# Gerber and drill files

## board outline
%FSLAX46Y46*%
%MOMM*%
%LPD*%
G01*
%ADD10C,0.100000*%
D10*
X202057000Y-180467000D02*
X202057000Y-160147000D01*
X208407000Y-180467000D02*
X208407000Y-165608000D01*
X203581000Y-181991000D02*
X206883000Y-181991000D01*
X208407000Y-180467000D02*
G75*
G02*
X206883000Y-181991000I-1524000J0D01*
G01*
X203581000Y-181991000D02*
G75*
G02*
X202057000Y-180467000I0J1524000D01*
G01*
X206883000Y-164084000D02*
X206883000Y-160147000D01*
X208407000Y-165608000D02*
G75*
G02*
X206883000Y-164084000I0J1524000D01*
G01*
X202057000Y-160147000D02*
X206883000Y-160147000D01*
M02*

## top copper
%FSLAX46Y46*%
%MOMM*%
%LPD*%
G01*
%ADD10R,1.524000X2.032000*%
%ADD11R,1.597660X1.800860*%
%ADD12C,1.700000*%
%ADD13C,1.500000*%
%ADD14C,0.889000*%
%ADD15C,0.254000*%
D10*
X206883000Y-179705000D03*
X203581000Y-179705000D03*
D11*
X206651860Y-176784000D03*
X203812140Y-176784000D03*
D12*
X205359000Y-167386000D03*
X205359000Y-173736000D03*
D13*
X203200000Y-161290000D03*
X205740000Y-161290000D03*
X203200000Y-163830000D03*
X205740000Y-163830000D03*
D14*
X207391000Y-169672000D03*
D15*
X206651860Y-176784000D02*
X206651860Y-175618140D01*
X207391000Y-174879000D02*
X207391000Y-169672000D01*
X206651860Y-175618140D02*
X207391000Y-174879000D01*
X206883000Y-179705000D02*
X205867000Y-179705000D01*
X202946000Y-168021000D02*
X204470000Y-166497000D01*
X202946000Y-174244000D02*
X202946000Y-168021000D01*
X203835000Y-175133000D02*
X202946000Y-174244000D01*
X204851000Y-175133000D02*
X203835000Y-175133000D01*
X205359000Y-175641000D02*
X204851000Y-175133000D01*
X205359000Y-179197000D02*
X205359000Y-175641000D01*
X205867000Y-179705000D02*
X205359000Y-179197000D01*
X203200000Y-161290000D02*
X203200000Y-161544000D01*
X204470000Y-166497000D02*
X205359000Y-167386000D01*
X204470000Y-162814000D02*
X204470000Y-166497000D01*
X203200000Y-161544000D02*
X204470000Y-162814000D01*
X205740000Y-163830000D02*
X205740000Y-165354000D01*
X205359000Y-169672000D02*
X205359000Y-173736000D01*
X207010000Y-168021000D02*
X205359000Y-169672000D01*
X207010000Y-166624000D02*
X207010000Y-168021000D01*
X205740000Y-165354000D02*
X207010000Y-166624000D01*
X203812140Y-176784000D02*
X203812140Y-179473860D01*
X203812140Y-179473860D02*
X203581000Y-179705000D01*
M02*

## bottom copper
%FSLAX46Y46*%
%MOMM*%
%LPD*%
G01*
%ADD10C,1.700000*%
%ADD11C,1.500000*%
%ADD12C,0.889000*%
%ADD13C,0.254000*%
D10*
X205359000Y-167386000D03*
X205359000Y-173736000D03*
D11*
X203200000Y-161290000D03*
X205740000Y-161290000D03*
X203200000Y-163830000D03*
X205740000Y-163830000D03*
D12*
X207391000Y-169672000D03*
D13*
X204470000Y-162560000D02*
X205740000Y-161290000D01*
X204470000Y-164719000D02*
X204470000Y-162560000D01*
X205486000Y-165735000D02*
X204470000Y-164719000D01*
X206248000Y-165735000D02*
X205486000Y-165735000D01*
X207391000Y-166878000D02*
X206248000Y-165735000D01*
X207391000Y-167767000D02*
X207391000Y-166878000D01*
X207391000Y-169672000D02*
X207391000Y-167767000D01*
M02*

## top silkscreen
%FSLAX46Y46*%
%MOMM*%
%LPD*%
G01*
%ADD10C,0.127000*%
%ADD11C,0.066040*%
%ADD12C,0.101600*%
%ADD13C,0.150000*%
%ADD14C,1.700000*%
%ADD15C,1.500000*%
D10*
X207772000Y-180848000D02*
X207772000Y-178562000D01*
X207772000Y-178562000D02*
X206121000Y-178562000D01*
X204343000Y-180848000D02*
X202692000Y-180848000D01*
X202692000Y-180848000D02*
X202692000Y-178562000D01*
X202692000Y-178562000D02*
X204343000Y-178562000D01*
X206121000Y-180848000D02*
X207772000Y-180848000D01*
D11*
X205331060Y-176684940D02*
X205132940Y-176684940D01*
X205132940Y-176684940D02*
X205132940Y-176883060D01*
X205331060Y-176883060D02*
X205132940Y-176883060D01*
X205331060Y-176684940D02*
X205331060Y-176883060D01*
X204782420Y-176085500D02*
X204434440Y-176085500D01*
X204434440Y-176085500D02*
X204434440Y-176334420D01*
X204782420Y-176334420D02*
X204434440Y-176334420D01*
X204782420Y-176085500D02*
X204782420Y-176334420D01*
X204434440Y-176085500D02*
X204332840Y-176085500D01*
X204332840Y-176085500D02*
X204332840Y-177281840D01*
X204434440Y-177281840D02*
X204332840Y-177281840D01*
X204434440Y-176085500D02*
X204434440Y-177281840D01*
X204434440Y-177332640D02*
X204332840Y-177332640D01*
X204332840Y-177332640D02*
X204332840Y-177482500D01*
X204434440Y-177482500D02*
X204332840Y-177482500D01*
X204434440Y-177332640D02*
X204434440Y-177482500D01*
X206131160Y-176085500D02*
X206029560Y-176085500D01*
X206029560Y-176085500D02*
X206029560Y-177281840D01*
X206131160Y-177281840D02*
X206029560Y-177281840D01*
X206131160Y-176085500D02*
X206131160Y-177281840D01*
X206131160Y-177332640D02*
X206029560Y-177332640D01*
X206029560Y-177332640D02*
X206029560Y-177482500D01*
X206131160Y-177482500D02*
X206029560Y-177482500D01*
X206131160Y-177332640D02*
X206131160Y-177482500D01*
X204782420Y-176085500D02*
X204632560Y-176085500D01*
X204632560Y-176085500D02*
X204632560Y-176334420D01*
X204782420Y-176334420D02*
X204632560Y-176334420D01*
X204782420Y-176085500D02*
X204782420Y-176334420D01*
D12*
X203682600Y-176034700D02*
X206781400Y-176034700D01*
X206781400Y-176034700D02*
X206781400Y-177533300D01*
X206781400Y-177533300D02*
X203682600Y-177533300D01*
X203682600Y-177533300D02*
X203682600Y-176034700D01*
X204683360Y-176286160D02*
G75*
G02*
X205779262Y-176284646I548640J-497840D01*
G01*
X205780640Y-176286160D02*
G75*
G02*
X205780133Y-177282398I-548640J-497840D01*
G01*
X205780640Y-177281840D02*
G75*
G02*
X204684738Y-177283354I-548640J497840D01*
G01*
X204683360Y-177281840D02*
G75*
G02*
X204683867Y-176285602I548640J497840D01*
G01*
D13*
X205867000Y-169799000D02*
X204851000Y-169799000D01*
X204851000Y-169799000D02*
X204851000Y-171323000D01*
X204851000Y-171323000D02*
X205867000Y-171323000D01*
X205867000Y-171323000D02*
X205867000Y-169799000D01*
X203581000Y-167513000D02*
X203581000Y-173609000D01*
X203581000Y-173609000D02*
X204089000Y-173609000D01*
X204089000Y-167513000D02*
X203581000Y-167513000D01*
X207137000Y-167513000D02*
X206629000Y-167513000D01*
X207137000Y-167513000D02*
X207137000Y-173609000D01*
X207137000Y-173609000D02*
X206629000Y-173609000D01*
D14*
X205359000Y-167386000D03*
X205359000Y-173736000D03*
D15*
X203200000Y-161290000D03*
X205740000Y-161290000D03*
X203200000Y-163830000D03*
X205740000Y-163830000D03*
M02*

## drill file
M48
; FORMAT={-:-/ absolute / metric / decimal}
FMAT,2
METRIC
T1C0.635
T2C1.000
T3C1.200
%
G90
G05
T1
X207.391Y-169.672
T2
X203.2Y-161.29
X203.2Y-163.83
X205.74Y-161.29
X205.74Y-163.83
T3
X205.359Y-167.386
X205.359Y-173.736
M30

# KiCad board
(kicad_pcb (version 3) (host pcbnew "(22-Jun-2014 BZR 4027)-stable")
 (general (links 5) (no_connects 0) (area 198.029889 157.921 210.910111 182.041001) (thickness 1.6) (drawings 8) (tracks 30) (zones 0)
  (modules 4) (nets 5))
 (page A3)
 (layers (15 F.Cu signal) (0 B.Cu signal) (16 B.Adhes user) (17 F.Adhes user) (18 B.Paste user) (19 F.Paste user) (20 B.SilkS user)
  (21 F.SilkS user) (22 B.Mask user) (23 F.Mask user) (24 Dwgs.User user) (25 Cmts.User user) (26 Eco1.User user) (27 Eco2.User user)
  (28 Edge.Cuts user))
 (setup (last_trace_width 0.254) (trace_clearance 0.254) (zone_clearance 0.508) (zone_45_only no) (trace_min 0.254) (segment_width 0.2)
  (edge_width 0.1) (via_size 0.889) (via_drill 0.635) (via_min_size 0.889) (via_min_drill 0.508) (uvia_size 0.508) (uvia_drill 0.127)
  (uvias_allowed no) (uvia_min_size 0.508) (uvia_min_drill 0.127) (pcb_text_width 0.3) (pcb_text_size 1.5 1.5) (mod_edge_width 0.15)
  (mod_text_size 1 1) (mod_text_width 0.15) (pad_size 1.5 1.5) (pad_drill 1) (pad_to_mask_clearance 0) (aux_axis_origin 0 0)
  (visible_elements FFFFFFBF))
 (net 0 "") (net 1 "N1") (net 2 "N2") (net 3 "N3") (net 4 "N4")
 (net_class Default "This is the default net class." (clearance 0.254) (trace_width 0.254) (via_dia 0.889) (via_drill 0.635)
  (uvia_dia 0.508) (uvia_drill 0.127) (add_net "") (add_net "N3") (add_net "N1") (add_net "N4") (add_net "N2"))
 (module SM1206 (layer F.Cu) (at 205.232 179.705 180)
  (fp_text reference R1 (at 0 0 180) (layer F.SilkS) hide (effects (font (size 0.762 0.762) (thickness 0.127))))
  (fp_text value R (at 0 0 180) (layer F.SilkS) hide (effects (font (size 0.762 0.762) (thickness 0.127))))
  (fp_line (start -2.54 -1.143) (end -2.54 1.143) (layer F.SilkS) (width 0.127))
  (fp_line (start -2.54 1.143) (end -0.889 1.143) (layer F.SilkS) (width 0.127))
  (fp_line (start 0.889 -1.143) (end 2.54 -1.143) (layer F.SilkS) (width 0.127))
  (fp_line (start 2.54 -1.143) (end 2.54 1.143) (layer F.SilkS) (width 0.127))
  (fp_line (start 2.54 1.143) (end 0.889 1.143) (layer F.SilkS) (width 0.127))
  (fp_line (start -0.889 -1.143) (end -2.54 -1.143) (layer F.SilkS) (width 0.127))
  (pad 1 smd rect (at -1.651 0 180) (size 1.524 2.032) (layers F.Cu F.Paste F.Mask) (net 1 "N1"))
  (pad 2 smd rect (at 1.651 0 180) (size 1.524 2.032) (layers F.Cu F.Paste F.Mask) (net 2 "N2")))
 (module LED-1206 (layer F.Cu) (at 205.232 176.784 180)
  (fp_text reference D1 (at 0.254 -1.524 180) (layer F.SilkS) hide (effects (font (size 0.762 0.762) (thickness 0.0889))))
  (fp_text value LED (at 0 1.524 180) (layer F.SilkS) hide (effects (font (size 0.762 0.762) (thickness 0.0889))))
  (fp_line (start -0.09906 0.09906) (end 0.09906 0.09906) (layer F.SilkS) (width 0.06604))
  (fp_line (start 0.09906 0.09906) (end 0.09906 -0.09906) (layer F.SilkS) (width 0.06604))
  (fp_line (start -0.09906 -0.09906) (end 0.09906 -0.09906) (layer F.SilkS) (width 0.06604))
  (fp_line (start -0.09906 0.09906) (end -0.09906 -0.09906) (layer F.SilkS) (width 0.06604))
  (fp_line (start 0.44958 0.6985) (end 0.79756 0.6985) (layer F.SilkS) (width 0.06604))
  (fp_line (start 0.79756 0.6985) (end 0.79756 0.44958) (layer F.SilkS) (width 0.06604))
  (fp_line (start 0.44958 0.44958) (end 0.79756 0.44958) (layer F.SilkS) (width 0.06604))
  (fp_line (start 0.44958 0.6985) (end 0.44958 0.44958) (layer F.SilkS) (width 0.06604))
  (fp_line (start 0.79756 0.6985) (end 0.89916 0.6985) (layer F.SilkS) (width 0.06604))
  (fp_line (start 0.89916 0.6985) (end 0.89916 -0.49784) (layer F.SilkS) (width 0.06604))
  (fp_line (start 0.79756 -0.49784) (end 0.89916 -0.49784) (layer F.SilkS) (width 0.06604))
  (fp_line (start 0.79756 0.6985) (end 0.79756 -0.49784) (layer F.SilkS) (width 0.06604))
  (fp_line (start 0.79756 -0.54864) (end 0.89916 -0.54864) (layer F.SilkS) (width 0.06604))
  (fp_line (start 0.89916 -0.54864) (end 0.89916 -0.6985) (layer F.SilkS) (width 0.06604))
  (fp_line (start 0.79756 -0.6985) (end 0.89916 -0.6985) (layer F.SilkS) (width 0.06604))
  (fp_line (start 0.79756 -0.54864) (end 0.79756 -0.6985) (layer F.SilkS) (width 0.06604))
  (fp_line (start -0.89916 0.6985) (end -0.79756 0.6985) (layer F.SilkS) (width 0.06604))
  (fp_line (start -0.79756 0.6985) (end -0.79756 -0.49784) (layer F.SilkS) (width 0.06604))
  (fp_line (start -0.89916 -0.49784) (end -0.79756 -0.49784) (layer F.SilkS) (width 0.06604))
  (fp_line (start -0.89916 0.6985) (end -0.89916 -0.49784) (layer F.SilkS) (width 0.06604))
  (fp_line (start -0.89916 -0.54864) (end -0.79756 -0.54864) (layer F.SilkS) (width 0.06604))
  (fp_line (start -0.79756 -0.54864) (end -0.79756 -0.6985) (layer F.SilkS) (width 0.06604))
  (fp_line (start -0.89916 -0.6985) (end -0.79756 -0.6985) (layer F.SilkS) (width 0.06604))
  (fp_line (start -0.89916 -0.54864) (end -0.89916 -0.6985) (layer F.SilkS) (width 0.06604))
  (fp_line (start 0.44958 0.6985) (end 0.59944 0.6985) (layer F.SilkS) (width 0.06604))
  (fp_line (start 0.59944 0.6985) (end 0.59944 0.44958) (layer F.SilkS) (width 0.06604))
  (fp_line (start 0.44958 0.44958) (end 0.59944 0.44958) (layer F.SilkS) (width 0.06604))
  (fp_line (start 0.44958 0.6985) (end 0.44958 0.44958) (layer F.SilkS) (width 0.06604))
  (fp_line (start 1.5494 0.7493) (end -1.5494 0.7493) (layer F.SilkS) (width 0.1016))
  (fp_line (start -1.5494 0.7493) (end -1.5494 -0.7493) (layer F.SilkS) (width 0.1016))
  (fp_line (start -1.5494 -0.7493) (end 1.5494 -0.7493) (layer F.SilkS) (width 0.1016))
  (fp_line (start 1.5494 -0.7493) (end 1.5494 0.7493) (layer F.SilkS) (width 0.1016))
  (fp_arc (start 0 0) (end 0.54864 0.49784) (angle 95.4) (layer F.SilkS) (width 0.1016))
  (fp_arc (start 0 0) (end -0.54864 0.49784) (angle 84.5) (layer F.SilkS) (width 0.1016))
  (fp_arc (start 0 0) (end -0.54864 -0.49784) (angle 95.4) (layer F.SilkS) (width 0.1016))
  (fp_arc (start 0 0) (end 0.54864 -0.49784) (angle 84.5) (layer F.SilkS) (width 0.1016))
  (pad 1 smd rect (at -1.41986 0 180) (size 1.59766 1.80086) (layers F.Cu F.Paste F.Mask) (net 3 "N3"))
  (pad 2 smd rect (at 1.41986 0 180) (size 1.59766 1.80086) (layers F.Cu F.Paste F.Mask) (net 2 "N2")))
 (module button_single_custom (layer F.Cu) (at 205.359 170.561 270)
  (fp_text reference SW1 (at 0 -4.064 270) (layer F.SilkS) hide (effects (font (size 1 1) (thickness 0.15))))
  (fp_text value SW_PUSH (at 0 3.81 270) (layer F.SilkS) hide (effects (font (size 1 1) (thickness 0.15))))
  (fp_line (start -0.762 -0.508) (end -0.762 0.508) (layer F.SilkS) (width 0.15))
  (fp_line (start -0.762 0.508) (end 0.762 0.508) (layer F.SilkS) (width 0.15))
  (fp_line (start 0.762 0.508) (end 0.762 -0.508) (layer F.SilkS) (width 0.15))
  (fp_line (start 0.762 -0.508) (end -0.762 -0.508) (layer F.SilkS) (width 0.15))
  (fp_line (start -3.048 1.778) (end 3.048 1.778) (layer F.SilkS) (width 0.15))
  (fp_line (start 3.048 1.778) (end 3.048 1.27) (layer F.SilkS) (width 0.15))
  (fp_line (start -3.048 1.27) (end -3.048 1.778) (layer F.SilkS) (width 0.15))
  (fp_line (start -3.048 -1.778) (end -3.048 -1.27) (layer F.SilkS) (width 0.15))
  (fp_line (start -3.048 -1.778) (end 3.048 -1.778) (layer F.SilkS) (width 0.15))
  (fp_line (start 3.048 -1.778) (end 3.048 -1.27) (layer F.SilkS) (width 0.15))
  (pad 1 thru_hole circle (at -3.175 0 270) (size 1.7 1.7) (drill 1.2) (layers *.Cu *.Mask F.SilkS) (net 1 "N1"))
  (pad 2 thru_hole circle (at 3.175 0 270) (size 1.7 1.7) (drill 1.2) (layers *.Cu *.Mask F.SilkS) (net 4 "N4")))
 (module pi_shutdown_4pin (layer F.Cu) (at 204.47 162.56)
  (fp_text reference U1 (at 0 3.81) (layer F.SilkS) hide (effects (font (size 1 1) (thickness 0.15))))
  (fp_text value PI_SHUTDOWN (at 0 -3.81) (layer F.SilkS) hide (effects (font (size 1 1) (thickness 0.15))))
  (pad 14 thru_hole circle (at -1.27 -1.27) (size 1.5 1.5) (drill 1) (layers *.Cu *.Mask F.SilkS) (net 1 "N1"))
  (pad 16 thru_hole circle (at 1.27 -1.27) (size 1.5 1.5) (drill 1) (layers *.Cu *.Mask F.SilkS) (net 3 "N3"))
  (pad 13 thru_hole circle (at -1.27 1.27) (size 1.5 1.5) (drill 1) (layers *.Cu *.Mask F.SilkS))
  (pad 15 thru_hole circle (at 1.27 1.27) (size 1.5 1.5) (drill 1) (layers *.Cu *.Mask F.SilkS) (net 4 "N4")))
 (gr_line (start 202.057 180.467) (end 202.057 160.147) (angle 90) (layer Edge.Cuts) (width 0.1))
 (gr_line (start 208.407 180.467) (end 208.407 165.608) (angle 90) (layer Edge.Cuts) (width 0.1))
 (gr_line (start 203.581 181.991) (end 206.883 181.991) (angle 90) (layer Edge.Cuts) (width 0.1))
 (gr_arc (start 206.883 180.467) (end 208.407 180.467) (angle 90) (layer Edge.Cuts) (width 0.1))
 (gr_arc (start 203.581 180.467) (end 203.581 181.991) (angle 90) (layer Edge.Cuts) (width 0.1))
 (gr_line (start 206.883 164.084) (end 206.883 160.147) (angle 90) (layer Edge.Cuts) (width 0.1))
 (gr_arc (start 208.407 164.084) (end 208.407 165.608) (angle 90) (layer Edge.Cuts) (width 0.1))
 (gr_line (start 202.057 160.147) (end 206.883 160.147) (angle 90) (layer Edge.Cuts) (width 0.1))
 (segment (start 206.65186 176.784) (end 206.65186 175.61814) (width 0.254) (layer F.Cu) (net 3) (status 400000))
 (segment (start 204.47 162.56) (end 205.74 161.29) (width 0.254) (layer B.Cu) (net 3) (status 800000))
 (segment (start 204.47 164.719) (end 204.47 162.56) (width 0.254) (layer B.Cu) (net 3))
 (segment (start 205.486 165.735) (end 204.47 164.719) (width 0.254) (layer B.Cu) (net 3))
 (segment (start 206.248 165.735) (end 205.486 165.735) (width 0.254) (layer B.Cu) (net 3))
 (segment (start 207.391 166.878) (end 206.248 165.735) (width 0.254) (layer B.Cu) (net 3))
 (segment (start 207.391 167.767) (end 207.391 166.878) (width 0.254) (layer B.Cu) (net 3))
 (segment (start 207.391 169.672) (end 207.391 167.767) (width 0.254) (layer B.Cu) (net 3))
 (via (at 207.391 169.672) (size 0.889) (layers F.Cu B.Cu) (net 3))
 (segment (start 207.391 174.879) (end 207.391 169.672) (width 0.254) (layer F.Cu) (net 3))
 (segment (start 206.65186 175.61814) (end 207.391 174.879) (width 0.254) (layer F.Cu) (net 3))
 (segment (start 206.883 179.705) (end 205.867 179.705) (width 0.254) (layer F.Cu) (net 1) (status 400000))
 (segment (start 202.946 168.021) (end 204.47 166.497) (width 0.254) (layer F.Cu) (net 1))
 (segment (start 202.946 174.244) (end 202.946 168.021) (width 0.254) (layer F.Cu) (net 1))
 (segment (start 203.835 175.133) (end 202.946 174.244) (width 0.254) (layer F.Cu) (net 1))
 (segment (start 204.851 175.133) (end 203.835 175.133) (width 0.254) (layer F.Cu) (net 1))
 (segment (start 205.359 175.641) (end 204.851 175.133) (width 0.254) (layer F.Cu) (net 1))
 (segment (start 205.359 179.197) (end 205.359 175.641) (width 0.254) (layer F.Cu) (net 1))
 (segment (start 205.867 179.705) (end 205.359 179.197) (width 0.254) (layer F.Cu) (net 1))
 (segment (start 203.2 161.29) (end 203.2 161.544) (width 0.254) (layer F.Cu) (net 1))
 (segment (start 204.47 166.497) (end 205.359 167.386) (width 0.254) (layer F.Cu) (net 1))
 (segment (start 204.47 162.814) (end 204.47 166.497) (width 0.254) (layer F.Cu) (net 1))
 (segment (start 203.2 161.544) (end 204.47 162.814) (width 0.254) (layer F.Cu) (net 1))
 (segment (start 205.74 163.83) (end 205.74 165.354) (width 0.254) (layer F.Cu) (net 4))
 (segment (start 205.359 169.672) (end 205.359 173.736) (width 0.254) (layer F.Cu) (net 4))
 (segment (start 207.01 168.021) (end 205.359 169.672) (width 0.254) (layer F.Cu) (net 4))
 (segment (start 207.01 166.624) (end 207.01 168.021) (width 0.254) (layer F.Cu) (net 4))
 (segment (start 205.74 165.354) (end 207.01 166.624) (width 0.254) (layer F.Cu) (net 4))
 (segment (start 203.81214 176.784) (end 203.81214 179.47386) (width 0.254) (layer F.Cu) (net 2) (status C00000))
 (segment (start 203.81214 179.47386) (end 203.581 179.705) (width 0.254) (layer F.Cu) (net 2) (status C00000)))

